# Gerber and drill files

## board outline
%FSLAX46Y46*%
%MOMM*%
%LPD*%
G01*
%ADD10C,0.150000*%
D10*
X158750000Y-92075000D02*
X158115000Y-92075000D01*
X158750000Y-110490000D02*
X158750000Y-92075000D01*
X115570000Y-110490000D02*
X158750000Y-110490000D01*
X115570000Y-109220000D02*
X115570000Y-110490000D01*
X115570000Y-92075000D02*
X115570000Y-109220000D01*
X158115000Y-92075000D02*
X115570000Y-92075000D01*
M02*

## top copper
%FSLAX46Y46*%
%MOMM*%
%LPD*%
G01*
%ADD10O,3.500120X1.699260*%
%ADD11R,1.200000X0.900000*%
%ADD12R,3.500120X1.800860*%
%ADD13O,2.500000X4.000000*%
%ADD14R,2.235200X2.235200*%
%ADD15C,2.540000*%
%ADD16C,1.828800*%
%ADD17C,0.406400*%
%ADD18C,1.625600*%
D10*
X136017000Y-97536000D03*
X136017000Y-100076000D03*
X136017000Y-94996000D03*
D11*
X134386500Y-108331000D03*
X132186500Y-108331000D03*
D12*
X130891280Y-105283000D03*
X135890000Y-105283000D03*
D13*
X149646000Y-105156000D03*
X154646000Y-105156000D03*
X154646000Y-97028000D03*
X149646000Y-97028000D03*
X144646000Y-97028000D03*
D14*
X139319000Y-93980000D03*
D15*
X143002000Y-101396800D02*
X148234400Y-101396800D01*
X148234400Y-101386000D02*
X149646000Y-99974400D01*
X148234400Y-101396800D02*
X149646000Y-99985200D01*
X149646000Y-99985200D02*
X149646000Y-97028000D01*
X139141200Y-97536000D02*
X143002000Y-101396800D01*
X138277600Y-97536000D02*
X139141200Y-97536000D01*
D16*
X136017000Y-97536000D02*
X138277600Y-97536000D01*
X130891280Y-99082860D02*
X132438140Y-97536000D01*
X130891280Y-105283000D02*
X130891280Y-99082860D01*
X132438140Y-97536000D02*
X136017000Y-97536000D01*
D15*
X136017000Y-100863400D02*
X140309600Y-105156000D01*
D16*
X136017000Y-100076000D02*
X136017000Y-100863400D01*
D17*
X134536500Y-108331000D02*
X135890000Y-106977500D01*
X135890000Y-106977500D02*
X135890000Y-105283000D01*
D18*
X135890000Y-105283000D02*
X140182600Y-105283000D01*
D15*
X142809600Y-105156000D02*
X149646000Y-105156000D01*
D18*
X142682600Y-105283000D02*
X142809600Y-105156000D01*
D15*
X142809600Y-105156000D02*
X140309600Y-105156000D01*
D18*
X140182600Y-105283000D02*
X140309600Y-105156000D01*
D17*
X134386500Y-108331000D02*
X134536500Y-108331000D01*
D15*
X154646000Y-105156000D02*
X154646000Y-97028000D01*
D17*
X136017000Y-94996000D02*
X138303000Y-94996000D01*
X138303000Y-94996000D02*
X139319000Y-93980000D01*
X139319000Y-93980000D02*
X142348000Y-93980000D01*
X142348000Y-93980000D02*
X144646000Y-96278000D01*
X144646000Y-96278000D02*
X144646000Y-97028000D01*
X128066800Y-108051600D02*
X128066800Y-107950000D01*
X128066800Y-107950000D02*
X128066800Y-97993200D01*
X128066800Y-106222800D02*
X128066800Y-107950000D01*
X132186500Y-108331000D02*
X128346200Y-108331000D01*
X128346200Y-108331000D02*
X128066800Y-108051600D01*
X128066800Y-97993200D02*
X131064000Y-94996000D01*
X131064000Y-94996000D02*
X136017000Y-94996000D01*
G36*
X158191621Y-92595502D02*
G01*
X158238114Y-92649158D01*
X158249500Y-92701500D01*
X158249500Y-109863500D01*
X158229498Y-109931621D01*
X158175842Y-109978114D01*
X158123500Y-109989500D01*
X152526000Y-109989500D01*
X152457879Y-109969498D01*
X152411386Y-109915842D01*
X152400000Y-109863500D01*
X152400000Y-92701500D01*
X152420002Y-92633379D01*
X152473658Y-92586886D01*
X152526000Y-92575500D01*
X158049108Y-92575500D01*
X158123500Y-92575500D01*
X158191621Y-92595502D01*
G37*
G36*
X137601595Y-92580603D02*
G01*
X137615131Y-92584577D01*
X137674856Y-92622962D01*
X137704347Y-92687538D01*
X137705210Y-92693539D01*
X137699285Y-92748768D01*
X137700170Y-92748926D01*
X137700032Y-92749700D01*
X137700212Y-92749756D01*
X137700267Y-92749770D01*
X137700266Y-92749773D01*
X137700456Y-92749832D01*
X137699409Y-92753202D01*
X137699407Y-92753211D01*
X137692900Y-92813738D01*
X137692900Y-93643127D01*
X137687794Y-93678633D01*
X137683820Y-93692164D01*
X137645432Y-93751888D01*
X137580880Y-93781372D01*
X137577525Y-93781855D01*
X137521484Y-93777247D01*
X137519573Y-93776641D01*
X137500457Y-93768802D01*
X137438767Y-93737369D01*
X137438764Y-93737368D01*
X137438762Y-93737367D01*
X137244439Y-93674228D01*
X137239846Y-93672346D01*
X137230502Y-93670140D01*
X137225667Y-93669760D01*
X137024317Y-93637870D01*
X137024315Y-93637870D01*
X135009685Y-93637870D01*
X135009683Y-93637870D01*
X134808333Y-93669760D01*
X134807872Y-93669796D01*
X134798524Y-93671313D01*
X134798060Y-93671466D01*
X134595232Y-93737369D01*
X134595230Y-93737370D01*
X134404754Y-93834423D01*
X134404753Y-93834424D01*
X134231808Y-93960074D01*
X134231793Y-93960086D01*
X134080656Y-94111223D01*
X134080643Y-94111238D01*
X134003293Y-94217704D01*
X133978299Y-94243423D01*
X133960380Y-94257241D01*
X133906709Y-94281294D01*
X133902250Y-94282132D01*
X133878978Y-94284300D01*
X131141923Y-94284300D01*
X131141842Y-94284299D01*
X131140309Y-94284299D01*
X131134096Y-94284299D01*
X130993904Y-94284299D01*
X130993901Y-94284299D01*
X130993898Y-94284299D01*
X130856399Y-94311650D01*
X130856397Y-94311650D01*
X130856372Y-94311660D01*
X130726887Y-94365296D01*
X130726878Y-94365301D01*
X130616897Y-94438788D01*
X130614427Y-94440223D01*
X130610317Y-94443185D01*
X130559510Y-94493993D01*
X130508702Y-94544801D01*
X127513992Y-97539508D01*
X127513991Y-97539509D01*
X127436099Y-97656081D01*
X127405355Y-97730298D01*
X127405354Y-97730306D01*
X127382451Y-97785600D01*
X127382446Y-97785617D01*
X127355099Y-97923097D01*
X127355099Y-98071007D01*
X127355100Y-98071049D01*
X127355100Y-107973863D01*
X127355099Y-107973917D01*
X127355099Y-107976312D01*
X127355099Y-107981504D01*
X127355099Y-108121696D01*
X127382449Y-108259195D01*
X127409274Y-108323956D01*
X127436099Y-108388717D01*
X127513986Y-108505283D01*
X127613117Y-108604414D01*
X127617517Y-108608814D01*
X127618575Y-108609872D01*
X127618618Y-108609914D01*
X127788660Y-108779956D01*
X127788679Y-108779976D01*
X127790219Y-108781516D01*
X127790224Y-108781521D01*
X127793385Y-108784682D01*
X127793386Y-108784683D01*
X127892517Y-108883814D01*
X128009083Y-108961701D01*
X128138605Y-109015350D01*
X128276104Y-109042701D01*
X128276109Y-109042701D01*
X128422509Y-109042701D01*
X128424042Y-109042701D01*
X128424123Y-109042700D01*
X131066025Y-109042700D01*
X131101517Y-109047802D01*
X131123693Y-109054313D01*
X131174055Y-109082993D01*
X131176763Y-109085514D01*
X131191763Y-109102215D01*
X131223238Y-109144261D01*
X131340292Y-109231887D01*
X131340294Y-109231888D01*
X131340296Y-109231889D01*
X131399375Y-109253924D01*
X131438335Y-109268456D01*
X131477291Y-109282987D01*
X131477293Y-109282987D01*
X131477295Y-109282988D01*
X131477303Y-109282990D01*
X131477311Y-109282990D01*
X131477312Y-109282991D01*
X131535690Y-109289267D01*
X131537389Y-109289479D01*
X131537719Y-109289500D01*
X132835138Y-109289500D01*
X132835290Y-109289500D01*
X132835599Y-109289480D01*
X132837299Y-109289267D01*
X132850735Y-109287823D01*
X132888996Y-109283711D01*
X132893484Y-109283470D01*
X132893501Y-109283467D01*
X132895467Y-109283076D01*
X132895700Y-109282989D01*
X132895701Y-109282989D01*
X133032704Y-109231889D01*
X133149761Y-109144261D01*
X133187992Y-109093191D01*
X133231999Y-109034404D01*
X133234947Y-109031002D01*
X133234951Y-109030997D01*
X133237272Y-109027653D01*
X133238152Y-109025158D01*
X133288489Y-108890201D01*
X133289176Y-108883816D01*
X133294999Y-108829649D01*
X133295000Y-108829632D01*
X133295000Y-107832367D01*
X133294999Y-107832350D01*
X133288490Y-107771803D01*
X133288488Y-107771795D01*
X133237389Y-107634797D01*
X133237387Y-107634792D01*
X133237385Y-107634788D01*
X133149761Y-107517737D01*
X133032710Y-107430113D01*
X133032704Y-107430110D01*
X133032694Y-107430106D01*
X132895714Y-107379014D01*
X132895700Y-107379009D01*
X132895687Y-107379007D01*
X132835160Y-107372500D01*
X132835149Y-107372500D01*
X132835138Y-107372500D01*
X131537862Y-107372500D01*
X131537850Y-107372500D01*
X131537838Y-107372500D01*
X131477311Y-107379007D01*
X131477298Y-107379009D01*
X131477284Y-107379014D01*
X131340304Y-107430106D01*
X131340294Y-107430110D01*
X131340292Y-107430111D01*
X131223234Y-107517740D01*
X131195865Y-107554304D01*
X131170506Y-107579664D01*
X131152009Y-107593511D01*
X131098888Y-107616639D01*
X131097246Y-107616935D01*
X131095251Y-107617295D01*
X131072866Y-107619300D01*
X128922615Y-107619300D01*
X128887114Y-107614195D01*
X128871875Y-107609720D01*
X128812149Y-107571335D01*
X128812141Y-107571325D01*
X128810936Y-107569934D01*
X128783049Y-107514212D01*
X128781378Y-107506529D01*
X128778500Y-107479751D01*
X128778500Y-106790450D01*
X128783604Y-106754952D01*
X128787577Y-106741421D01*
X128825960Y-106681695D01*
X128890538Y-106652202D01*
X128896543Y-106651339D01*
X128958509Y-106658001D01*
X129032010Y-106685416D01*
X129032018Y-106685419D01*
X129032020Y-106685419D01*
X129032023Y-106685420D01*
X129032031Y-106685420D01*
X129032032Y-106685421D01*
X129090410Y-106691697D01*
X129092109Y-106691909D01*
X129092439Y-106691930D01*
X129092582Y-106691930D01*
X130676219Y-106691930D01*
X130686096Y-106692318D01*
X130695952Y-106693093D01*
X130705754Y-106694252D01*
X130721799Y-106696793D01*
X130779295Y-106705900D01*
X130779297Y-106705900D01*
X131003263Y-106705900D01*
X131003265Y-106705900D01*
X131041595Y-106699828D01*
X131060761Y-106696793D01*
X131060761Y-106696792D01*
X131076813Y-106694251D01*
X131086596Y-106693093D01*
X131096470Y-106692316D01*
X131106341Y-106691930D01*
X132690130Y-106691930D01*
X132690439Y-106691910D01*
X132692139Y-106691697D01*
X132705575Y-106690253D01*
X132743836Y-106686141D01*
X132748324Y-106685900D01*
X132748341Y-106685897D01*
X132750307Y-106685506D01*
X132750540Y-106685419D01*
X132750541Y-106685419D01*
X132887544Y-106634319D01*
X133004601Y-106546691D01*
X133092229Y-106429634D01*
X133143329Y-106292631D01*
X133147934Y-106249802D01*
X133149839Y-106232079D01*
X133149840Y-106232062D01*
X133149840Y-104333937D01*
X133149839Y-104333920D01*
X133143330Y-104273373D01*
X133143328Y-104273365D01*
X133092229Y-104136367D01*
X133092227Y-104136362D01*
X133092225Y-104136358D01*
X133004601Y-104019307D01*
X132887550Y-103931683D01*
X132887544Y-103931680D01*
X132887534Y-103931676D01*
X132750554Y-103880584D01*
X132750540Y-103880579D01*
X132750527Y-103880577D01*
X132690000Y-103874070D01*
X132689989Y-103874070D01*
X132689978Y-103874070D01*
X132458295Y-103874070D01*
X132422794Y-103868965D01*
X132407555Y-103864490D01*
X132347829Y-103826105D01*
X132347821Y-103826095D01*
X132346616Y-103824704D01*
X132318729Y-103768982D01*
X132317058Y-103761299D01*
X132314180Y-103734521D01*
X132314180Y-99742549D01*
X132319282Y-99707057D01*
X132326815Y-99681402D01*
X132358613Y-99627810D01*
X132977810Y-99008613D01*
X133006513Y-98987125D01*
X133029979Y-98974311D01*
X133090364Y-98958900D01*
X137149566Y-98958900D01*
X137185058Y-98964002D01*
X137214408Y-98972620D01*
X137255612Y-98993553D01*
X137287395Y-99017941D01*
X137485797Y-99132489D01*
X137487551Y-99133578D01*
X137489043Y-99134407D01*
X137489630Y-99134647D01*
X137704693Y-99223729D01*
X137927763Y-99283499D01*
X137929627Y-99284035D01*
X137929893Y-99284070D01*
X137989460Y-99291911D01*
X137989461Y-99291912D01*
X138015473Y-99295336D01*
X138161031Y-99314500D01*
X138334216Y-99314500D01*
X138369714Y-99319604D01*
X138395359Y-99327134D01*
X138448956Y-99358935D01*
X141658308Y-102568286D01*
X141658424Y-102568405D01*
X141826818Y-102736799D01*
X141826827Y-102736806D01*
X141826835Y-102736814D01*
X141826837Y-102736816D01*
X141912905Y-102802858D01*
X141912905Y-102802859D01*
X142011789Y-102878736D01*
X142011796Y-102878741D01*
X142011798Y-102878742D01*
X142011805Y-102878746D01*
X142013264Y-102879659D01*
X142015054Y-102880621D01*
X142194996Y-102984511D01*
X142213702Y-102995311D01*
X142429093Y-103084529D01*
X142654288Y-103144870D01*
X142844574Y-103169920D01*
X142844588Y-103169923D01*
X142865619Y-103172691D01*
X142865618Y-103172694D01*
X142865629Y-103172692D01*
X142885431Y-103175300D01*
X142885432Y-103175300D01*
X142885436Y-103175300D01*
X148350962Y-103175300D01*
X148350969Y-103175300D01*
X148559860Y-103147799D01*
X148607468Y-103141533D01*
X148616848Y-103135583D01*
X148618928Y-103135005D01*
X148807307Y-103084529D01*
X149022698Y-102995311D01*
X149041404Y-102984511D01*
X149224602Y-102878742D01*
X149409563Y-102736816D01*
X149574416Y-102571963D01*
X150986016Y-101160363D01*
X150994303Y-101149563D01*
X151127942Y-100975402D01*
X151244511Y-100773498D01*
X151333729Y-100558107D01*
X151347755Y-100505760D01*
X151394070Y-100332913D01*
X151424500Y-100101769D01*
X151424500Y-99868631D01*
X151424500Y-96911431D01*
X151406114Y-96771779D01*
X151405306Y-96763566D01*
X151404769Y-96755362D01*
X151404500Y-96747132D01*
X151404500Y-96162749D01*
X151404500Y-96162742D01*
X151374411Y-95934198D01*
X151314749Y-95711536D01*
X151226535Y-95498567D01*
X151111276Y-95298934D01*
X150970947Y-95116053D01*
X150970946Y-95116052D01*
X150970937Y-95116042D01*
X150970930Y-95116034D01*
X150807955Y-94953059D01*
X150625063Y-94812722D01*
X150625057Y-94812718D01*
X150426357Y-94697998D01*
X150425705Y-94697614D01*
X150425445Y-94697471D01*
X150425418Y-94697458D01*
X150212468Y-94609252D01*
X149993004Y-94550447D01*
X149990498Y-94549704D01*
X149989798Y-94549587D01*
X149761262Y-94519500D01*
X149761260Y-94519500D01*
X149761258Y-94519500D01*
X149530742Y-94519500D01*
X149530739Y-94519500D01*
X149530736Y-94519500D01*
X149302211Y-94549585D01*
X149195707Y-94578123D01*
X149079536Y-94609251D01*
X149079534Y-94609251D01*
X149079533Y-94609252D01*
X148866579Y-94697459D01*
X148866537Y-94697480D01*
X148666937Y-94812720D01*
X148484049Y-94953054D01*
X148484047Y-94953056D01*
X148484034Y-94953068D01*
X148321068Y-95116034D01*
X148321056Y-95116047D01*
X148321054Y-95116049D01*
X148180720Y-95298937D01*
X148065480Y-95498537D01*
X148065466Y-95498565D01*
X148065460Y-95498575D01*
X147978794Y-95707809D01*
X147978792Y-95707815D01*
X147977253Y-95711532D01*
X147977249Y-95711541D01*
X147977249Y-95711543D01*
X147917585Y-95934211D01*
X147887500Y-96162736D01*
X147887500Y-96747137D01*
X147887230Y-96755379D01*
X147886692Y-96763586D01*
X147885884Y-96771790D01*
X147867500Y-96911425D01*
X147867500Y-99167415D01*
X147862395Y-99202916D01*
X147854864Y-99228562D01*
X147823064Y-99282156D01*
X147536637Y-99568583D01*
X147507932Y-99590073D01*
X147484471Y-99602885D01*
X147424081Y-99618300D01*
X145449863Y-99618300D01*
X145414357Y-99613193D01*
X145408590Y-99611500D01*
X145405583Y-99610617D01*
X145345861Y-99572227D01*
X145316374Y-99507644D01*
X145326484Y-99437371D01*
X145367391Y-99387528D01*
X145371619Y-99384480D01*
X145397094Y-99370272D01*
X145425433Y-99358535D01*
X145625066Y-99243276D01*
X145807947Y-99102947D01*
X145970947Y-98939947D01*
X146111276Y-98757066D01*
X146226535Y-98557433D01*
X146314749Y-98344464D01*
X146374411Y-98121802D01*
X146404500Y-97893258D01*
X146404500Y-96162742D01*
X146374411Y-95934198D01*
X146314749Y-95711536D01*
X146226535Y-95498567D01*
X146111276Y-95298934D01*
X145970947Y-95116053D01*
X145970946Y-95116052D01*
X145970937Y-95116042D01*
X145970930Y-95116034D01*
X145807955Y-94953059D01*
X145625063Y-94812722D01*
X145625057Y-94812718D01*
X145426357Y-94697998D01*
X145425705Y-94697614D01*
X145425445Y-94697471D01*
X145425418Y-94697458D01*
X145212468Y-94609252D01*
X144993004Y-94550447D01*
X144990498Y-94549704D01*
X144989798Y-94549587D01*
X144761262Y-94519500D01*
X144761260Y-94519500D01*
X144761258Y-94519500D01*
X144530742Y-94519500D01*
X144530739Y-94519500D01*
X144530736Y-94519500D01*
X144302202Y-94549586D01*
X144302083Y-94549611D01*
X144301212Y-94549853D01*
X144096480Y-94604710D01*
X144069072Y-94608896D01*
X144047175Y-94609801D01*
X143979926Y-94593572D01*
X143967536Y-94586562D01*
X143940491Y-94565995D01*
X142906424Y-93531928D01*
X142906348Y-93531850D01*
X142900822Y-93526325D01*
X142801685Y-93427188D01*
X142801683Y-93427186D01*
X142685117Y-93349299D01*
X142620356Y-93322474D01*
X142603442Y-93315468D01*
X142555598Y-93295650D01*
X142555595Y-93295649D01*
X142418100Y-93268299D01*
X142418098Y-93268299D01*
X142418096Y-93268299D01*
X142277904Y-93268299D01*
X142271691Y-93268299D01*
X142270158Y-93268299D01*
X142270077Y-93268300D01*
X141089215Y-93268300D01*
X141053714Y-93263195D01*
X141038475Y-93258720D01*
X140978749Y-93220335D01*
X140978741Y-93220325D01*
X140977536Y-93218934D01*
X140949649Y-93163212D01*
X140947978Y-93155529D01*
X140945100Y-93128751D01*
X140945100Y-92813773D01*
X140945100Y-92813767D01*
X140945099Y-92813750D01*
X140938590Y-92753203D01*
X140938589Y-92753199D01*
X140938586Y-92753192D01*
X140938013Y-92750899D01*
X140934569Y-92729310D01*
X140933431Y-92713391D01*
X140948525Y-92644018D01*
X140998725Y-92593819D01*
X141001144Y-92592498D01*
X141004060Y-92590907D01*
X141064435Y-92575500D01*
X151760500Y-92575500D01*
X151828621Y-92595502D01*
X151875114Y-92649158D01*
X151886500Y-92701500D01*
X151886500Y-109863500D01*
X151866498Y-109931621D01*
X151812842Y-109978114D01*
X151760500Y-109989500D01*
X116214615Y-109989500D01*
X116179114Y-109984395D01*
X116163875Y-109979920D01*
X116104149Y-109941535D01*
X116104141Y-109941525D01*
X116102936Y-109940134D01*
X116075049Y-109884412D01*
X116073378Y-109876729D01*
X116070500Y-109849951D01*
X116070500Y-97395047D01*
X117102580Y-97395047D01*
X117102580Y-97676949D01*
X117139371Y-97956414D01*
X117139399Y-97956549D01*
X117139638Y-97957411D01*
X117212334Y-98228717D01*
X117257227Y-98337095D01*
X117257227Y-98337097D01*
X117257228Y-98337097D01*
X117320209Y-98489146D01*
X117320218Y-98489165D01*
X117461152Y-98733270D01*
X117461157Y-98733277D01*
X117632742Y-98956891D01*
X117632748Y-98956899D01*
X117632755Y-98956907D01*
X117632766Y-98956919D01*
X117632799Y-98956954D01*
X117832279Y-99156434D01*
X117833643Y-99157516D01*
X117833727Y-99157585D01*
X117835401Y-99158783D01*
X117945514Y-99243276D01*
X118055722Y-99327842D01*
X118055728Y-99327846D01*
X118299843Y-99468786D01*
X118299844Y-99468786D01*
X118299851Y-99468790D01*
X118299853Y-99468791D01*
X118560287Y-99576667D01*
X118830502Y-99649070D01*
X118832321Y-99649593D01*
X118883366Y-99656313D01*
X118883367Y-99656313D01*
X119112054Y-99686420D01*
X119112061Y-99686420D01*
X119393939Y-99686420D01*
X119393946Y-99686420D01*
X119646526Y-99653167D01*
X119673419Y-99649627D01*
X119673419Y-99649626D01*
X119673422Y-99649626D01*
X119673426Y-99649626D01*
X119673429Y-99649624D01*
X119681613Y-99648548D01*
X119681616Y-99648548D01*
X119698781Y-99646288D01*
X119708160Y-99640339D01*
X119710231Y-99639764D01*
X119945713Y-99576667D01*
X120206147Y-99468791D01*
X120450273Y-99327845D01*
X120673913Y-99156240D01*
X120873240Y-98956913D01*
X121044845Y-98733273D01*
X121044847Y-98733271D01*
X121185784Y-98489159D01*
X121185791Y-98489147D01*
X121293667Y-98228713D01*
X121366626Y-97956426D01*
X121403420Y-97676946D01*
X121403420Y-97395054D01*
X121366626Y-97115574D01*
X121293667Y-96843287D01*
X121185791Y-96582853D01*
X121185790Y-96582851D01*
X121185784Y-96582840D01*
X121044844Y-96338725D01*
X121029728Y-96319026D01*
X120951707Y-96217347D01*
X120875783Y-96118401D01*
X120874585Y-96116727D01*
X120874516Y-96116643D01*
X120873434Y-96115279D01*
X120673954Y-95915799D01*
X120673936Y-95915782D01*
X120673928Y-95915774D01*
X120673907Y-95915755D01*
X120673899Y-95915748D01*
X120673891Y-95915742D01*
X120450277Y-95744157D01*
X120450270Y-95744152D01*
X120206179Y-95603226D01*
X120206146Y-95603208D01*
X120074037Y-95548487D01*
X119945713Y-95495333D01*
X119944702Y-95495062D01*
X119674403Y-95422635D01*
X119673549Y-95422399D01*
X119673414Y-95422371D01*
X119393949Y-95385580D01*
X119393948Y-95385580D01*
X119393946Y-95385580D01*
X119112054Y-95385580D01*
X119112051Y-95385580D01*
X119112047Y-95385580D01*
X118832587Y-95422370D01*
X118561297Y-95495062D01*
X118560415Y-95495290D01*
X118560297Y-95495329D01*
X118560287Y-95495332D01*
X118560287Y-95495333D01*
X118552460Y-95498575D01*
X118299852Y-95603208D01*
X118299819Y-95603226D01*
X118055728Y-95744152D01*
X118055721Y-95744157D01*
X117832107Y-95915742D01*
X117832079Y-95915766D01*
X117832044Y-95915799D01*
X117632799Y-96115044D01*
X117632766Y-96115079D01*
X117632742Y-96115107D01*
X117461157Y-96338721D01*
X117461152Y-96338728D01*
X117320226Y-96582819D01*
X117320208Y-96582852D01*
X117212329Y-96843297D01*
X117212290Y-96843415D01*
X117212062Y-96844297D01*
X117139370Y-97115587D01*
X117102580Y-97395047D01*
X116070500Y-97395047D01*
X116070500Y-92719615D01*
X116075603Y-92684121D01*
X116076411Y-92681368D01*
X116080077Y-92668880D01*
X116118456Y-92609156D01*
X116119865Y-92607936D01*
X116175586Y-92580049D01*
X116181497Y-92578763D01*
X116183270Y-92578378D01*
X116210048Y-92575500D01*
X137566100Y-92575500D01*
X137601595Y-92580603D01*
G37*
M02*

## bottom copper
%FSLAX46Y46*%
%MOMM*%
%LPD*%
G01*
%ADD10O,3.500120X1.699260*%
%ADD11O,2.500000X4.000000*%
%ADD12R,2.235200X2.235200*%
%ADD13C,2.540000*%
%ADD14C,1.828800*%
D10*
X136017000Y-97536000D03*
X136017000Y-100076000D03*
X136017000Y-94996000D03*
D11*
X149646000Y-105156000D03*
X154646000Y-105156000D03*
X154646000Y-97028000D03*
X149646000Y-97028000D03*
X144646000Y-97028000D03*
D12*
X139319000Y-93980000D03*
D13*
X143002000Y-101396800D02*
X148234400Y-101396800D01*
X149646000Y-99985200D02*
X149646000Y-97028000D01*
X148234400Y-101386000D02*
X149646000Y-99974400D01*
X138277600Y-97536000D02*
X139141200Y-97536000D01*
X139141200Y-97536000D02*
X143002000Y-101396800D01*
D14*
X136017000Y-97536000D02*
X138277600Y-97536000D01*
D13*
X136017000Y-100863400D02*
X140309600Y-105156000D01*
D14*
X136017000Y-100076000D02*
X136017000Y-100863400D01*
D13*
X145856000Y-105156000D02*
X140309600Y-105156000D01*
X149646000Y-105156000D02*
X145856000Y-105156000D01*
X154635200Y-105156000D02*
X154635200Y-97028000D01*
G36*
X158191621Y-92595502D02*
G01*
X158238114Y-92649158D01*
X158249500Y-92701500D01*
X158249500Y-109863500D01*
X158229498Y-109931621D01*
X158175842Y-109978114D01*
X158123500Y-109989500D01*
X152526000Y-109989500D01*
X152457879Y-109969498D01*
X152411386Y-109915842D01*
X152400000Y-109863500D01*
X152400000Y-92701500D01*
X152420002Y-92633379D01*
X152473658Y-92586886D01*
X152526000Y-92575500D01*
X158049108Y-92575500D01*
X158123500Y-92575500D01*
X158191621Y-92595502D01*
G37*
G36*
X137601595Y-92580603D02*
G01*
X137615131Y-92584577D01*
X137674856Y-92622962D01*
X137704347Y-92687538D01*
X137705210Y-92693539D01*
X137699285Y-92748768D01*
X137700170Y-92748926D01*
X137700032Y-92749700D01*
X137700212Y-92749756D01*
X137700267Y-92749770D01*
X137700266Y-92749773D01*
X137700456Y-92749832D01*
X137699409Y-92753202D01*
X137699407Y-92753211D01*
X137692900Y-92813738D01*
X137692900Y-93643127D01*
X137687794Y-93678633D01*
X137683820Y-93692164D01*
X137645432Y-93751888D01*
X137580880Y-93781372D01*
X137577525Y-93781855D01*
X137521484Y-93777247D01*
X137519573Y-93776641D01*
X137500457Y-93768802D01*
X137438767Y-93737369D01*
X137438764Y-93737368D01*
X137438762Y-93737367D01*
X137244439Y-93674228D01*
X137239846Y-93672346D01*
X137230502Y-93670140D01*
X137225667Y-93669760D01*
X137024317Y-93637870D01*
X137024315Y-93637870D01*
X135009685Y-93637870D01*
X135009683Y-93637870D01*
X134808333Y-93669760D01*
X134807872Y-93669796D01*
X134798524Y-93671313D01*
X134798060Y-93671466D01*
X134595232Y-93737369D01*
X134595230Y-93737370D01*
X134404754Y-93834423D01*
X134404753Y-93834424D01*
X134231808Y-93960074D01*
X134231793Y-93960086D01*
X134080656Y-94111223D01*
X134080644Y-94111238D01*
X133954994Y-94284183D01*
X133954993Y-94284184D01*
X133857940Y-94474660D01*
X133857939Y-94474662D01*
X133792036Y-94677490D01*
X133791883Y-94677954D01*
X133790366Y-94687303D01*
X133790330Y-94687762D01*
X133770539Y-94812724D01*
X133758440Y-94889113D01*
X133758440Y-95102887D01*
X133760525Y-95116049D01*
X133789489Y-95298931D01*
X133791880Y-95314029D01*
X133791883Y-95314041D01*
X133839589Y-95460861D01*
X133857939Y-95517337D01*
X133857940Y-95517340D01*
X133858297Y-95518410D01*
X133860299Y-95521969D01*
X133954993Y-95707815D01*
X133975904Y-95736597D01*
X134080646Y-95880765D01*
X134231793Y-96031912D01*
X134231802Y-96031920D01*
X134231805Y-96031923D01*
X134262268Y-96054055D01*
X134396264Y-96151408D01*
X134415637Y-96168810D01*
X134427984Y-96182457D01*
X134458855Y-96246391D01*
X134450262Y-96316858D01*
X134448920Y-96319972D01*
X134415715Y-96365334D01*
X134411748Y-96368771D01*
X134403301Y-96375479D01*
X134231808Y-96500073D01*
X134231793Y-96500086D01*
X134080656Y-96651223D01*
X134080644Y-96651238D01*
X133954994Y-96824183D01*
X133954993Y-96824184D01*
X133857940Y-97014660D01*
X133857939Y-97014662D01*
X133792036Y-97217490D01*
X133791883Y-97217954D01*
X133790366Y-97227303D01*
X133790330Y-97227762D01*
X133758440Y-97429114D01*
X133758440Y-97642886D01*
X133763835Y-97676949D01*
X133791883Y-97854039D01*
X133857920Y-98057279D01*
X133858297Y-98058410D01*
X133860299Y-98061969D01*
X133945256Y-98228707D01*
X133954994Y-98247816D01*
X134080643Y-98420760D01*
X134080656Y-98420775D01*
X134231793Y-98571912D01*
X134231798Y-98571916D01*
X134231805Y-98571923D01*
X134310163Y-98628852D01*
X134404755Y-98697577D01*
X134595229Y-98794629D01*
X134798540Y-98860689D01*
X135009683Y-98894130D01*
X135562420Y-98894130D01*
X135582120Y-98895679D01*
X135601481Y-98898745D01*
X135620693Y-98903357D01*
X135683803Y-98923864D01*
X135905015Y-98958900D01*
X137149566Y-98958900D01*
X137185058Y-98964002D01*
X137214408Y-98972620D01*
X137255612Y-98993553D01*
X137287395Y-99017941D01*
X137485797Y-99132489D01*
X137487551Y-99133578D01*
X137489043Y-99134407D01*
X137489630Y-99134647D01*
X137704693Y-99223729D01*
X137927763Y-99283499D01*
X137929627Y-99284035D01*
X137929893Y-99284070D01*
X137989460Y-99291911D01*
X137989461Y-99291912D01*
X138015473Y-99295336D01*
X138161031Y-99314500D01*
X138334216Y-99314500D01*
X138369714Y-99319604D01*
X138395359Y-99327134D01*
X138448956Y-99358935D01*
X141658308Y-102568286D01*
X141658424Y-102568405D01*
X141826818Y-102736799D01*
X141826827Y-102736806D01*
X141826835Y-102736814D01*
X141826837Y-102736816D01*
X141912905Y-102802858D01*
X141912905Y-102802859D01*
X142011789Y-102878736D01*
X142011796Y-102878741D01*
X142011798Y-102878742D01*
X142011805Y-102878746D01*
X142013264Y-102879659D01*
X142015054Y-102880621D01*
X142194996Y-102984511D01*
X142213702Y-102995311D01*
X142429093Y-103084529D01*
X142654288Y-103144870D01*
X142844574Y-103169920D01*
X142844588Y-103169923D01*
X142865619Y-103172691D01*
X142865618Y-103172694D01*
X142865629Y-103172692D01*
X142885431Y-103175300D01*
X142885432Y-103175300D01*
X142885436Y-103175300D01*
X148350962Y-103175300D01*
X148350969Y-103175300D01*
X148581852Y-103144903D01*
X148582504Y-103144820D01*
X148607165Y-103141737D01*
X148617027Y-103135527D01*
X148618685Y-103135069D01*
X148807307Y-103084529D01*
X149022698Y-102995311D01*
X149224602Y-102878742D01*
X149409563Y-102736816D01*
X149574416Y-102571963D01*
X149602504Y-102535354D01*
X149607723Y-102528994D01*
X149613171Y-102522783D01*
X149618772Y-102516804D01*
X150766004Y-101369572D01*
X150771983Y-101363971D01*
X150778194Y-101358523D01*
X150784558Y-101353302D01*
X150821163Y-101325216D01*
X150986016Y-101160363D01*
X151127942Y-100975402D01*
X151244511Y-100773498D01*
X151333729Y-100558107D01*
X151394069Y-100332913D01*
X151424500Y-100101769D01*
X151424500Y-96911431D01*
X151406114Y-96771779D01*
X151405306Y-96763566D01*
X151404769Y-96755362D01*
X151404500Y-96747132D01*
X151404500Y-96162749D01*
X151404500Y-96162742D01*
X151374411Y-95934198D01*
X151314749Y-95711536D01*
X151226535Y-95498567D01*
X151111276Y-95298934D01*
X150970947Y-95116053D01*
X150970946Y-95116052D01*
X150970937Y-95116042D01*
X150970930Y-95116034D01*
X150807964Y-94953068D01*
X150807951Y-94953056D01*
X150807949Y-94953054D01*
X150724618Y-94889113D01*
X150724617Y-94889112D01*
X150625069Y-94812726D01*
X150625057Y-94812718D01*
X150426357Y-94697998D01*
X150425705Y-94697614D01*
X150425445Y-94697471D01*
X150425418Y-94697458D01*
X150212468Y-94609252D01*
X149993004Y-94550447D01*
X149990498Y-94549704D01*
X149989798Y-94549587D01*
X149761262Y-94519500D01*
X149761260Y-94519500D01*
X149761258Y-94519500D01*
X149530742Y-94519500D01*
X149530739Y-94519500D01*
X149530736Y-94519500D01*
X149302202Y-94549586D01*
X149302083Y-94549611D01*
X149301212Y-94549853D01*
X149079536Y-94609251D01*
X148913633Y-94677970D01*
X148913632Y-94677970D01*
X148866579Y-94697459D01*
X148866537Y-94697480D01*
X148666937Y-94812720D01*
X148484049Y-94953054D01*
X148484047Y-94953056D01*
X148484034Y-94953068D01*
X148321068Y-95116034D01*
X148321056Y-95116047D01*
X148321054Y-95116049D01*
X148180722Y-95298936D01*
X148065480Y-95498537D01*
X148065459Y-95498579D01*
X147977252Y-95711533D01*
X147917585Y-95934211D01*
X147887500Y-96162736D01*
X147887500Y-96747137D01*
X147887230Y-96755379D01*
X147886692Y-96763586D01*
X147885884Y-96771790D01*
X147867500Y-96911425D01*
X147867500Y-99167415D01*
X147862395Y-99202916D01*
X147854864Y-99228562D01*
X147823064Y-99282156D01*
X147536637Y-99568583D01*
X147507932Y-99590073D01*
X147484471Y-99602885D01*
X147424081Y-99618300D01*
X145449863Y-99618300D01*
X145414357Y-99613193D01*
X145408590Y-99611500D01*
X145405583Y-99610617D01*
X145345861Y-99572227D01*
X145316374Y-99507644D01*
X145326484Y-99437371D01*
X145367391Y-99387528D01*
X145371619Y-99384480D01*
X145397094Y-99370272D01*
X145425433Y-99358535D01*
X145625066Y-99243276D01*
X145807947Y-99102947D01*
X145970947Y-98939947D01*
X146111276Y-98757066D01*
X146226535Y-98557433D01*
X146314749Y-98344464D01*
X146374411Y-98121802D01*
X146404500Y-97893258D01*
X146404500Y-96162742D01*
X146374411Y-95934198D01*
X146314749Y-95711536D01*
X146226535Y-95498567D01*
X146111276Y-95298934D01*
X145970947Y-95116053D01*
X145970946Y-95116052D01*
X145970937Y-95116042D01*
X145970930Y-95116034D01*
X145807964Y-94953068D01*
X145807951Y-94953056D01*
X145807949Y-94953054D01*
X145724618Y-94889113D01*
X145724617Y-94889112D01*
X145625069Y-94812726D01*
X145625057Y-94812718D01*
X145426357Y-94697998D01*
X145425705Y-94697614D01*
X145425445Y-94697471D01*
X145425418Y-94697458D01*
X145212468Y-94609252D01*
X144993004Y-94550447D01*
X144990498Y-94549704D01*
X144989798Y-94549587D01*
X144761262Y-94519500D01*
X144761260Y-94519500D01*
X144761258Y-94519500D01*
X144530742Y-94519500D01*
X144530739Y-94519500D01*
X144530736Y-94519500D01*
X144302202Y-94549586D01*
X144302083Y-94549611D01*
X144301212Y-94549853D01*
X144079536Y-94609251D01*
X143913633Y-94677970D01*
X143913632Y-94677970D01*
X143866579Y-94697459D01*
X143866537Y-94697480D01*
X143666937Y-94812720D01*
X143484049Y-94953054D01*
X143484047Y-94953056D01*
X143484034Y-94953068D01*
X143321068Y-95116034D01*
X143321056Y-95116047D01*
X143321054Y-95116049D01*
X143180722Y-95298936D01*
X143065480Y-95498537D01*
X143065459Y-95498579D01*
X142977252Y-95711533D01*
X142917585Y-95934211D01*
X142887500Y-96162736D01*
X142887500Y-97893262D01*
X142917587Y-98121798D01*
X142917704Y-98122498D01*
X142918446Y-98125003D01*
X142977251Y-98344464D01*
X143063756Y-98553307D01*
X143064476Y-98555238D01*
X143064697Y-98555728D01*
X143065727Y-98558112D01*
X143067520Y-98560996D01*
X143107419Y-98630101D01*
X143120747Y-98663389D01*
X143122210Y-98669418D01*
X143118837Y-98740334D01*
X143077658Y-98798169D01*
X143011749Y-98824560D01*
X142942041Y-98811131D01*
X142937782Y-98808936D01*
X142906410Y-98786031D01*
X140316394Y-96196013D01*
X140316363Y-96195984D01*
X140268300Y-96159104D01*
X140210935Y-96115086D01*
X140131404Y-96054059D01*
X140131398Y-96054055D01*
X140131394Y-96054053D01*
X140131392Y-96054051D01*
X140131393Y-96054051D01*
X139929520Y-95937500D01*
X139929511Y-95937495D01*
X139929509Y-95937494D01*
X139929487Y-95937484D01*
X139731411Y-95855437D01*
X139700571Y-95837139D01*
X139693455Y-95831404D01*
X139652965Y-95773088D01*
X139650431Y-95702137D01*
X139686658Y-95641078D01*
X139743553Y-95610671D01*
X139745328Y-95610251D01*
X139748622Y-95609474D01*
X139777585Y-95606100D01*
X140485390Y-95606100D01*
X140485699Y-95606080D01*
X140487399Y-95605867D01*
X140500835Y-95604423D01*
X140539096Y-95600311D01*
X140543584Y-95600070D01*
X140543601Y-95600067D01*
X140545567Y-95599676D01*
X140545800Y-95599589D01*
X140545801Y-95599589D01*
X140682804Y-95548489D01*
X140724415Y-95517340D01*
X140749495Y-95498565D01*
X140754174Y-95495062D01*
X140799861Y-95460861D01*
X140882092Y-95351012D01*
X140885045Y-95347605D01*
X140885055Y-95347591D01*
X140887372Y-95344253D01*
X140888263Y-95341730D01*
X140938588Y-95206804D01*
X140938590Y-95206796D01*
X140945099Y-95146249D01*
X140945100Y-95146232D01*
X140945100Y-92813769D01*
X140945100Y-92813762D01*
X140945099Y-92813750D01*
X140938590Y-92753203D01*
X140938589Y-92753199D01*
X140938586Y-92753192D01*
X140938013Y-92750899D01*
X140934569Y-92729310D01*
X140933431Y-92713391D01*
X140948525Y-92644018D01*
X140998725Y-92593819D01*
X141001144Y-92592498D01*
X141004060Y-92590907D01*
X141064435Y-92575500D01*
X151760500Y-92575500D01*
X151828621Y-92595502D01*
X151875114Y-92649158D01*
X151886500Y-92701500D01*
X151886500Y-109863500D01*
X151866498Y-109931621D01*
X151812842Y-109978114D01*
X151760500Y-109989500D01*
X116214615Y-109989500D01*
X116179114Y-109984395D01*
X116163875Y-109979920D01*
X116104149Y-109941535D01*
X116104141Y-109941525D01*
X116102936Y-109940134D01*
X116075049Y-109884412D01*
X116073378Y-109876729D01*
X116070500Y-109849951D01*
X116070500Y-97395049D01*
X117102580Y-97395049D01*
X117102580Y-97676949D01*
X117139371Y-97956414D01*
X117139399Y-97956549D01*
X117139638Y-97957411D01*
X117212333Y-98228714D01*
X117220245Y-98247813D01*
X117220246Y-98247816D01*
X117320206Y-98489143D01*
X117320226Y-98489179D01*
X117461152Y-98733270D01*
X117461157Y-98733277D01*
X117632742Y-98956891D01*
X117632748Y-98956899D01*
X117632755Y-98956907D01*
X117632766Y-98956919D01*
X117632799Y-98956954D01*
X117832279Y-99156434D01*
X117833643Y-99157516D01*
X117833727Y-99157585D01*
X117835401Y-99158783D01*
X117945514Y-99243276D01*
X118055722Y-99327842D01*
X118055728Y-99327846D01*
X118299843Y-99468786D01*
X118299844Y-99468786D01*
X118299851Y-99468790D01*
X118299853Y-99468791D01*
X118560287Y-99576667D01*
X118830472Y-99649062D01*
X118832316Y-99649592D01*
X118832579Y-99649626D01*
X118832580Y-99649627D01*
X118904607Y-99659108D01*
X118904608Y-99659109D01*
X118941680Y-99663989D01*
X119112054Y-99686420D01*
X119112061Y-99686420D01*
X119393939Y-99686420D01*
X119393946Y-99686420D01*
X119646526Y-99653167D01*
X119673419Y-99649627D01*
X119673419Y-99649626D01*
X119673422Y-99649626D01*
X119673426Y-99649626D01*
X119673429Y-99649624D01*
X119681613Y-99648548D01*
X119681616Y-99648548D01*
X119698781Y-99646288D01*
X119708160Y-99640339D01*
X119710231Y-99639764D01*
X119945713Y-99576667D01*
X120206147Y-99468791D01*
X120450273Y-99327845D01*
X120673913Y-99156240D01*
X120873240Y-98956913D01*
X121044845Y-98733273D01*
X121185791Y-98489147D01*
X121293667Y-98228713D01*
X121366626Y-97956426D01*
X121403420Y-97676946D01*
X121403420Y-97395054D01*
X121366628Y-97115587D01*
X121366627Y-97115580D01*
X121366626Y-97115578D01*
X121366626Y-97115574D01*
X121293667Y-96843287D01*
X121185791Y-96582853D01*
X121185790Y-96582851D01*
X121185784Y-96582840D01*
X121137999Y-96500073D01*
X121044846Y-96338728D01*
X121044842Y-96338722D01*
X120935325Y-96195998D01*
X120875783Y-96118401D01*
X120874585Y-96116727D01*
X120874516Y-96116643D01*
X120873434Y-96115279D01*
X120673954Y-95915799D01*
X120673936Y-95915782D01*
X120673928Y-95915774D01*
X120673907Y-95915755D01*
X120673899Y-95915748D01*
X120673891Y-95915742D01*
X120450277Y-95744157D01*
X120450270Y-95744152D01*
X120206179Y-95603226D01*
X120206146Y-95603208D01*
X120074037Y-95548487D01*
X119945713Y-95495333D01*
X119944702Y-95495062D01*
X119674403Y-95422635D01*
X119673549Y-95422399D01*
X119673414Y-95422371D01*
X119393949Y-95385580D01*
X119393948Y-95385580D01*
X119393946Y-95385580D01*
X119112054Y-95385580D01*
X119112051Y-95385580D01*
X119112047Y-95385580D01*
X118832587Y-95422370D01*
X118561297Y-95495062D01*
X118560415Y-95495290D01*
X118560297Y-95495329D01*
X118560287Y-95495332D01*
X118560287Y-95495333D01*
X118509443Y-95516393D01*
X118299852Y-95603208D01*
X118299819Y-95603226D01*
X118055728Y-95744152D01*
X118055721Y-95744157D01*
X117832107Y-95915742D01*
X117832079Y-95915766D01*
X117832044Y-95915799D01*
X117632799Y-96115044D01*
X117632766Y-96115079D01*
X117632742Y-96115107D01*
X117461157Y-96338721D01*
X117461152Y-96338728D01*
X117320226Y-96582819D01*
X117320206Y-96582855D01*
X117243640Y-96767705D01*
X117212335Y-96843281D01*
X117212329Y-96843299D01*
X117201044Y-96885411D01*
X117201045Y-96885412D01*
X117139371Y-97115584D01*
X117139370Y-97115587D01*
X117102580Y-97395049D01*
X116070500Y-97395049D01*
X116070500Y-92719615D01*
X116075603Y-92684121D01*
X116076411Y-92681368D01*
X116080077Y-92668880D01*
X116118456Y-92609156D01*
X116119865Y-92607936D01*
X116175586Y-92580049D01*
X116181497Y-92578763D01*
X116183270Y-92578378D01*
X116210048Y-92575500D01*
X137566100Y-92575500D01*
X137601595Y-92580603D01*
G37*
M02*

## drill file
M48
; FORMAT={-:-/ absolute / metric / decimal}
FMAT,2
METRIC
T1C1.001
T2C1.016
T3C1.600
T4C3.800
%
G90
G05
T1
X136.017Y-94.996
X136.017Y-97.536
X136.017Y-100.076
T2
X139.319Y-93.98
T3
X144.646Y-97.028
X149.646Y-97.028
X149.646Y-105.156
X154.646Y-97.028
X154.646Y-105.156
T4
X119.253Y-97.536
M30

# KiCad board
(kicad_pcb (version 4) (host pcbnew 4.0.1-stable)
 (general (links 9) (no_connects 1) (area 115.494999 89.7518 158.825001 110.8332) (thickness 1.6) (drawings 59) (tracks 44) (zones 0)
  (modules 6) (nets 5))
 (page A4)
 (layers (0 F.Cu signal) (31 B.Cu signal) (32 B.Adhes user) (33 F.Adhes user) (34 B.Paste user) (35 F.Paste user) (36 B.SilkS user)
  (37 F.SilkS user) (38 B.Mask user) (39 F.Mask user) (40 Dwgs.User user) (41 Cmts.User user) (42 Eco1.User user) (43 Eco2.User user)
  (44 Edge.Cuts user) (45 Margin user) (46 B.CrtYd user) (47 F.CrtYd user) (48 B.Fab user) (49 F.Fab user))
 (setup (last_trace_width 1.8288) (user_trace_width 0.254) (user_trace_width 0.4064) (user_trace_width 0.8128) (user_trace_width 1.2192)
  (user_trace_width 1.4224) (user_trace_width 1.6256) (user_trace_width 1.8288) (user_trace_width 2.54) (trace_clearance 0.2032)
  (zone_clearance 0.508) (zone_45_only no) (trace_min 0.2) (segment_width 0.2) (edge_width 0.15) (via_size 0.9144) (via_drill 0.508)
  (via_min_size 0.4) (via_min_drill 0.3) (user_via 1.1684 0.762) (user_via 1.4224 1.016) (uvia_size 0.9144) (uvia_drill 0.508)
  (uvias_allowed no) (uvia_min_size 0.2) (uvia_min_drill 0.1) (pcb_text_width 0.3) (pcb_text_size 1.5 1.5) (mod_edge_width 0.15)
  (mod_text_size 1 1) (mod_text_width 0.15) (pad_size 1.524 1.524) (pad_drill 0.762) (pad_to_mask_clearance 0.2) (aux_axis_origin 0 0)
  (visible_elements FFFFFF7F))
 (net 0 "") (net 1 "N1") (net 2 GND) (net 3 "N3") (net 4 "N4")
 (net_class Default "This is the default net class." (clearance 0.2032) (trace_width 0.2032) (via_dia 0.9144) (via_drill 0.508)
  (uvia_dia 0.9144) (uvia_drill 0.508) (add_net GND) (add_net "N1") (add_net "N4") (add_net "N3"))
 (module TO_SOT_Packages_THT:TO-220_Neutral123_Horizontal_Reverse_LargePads (layer F.Cu) (at 136.017 97.536 90)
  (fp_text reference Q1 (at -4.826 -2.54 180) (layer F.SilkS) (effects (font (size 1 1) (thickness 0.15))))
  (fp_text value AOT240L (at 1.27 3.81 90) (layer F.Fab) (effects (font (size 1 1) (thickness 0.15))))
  (pad 2 thru_hole oval (at 0 0 180) (size 3.50012 1.69926) (drill 1.00076) (layers *.Cu *.Mask F.SilkS) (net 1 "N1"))
  (pad 3 thru_hole oval (at -2.54 0 180) (size 3.50012 1.69926) (drill 1.00076) (layers *.Cu *.Mask F.SilkS) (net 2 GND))
  (pad 1 thru_hole oval (at 2.54 0 180) (size 3.50012 1.69926) (drill 1.00076) (layers *.Cu *.Mask F.SilkS) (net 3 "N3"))
  (pad "" np_thru_hole circle (at 0 -16.764 180) (size 3.79984 3.79984) (drill 3.79984) (layers *.Cu *.Mask F.SilkS)))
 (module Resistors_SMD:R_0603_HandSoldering (layer F.Cu) (at 133.2865 108.331 180)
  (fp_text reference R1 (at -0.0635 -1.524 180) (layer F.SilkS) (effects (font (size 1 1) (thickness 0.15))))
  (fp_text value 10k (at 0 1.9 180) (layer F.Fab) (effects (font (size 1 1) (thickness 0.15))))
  (pad 1 smd rect (at -1.1 0 180) (size 1.2 0.9) (layers F.Cu F.Paste F.Mask) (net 2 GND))
  (pad 2 smd rect (at 1.1 0 180) (size 1.2 0.9) (layers F.Cu F.Paste F.Mask) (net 3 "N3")))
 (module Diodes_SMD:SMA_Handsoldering (layer F.Cu) (at 133.39064 105.283)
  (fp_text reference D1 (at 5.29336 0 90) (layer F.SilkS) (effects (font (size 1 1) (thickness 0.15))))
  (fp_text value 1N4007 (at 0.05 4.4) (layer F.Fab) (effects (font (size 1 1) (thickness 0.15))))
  (pad 1 smd rect (at -2.49936 0) (size 3.50012 1.80086) (layers F.Cu F.Paste F.Mask) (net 1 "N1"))
  (pad 2 smd rect (at 2.49936 0) (size 3.50012 1.80086) (layers F.Cu F.Paste F.Mask) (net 2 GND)))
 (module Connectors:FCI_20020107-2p (layer F.Cu) (at 152.146 105.156)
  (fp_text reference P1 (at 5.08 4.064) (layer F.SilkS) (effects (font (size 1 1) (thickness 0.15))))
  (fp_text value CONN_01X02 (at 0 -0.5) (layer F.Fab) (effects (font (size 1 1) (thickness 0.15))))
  (pad 1 thru_hole oval (at -2.5 0 180) (size 2.5 4) (drill 1.6) (layers *.Cu *.Mask F.SilkS) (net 2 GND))
  (pad 2 thru_hole oval (at 2.5 0) (size 2.5 4) (drill 1.6) (layers *.Cu *.Mask F.SilkS) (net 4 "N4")))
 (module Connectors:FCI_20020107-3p (layer F.Cu) (at 149.646 97.028 180)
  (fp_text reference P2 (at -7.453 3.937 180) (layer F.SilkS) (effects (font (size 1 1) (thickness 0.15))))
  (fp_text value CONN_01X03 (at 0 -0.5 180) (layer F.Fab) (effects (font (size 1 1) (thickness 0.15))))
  (pad 1 thru_hole oval (at -5 0) (size 2.5 4) (drill 1.6) (layers *.Cu *.Mask F.SilkS) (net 4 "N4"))
  (pad 2 thru_hole oval (at 0 0) (size 2.5 4) (drill 1.6) (layers *.Cu *.Mask F.SilkS) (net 1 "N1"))
  (pad 3 thru_hole oval (at 5 0) (size 2.5 4) (drill 1.6) (layers *.Cu *.Mask F.SilkS) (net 3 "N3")))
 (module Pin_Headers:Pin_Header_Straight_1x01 (layer F.Cu) (at 139.319 93.98)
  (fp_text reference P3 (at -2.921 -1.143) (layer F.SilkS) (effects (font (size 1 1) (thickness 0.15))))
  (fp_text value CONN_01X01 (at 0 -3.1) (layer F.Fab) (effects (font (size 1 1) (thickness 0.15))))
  (pad 1 thru_hole rect (at 0 0) (size 2.2352 2.2352) (drill 1.016) (layers *.Cu *.Mask F.SilkS) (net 3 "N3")))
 (gr_line (start 158.75 92.075) (end 158.115 92.075) (layer Edge.Cuts) (width 0.15))
 (gr_line (start 158.75 110.49) (end 158.75 92.075) (layer Edge.Cuts) (width 0.15))
 (gr_line (start 115.57 110.49) (end 158.75 110.49) (layer Edge.Cuts) (width 0.15))
 (gr_line (start 115.57 109.22) (end 115.57 110.49) (layer Edge.Cuts) (width 0.15))
 (gr_line (start 115.57 92.075) (end 115.57 109.22) (layer Edge.Cuts) (width 0.15))
 (gr_line (start 158.115 92.075) (end 115.57 92.075) (layer Edge.Cuts) (width 0.15))
 (segment (start 143.002 101.3968) (end 148.2344 101.3968) (width 2.54) (layer F.Cu) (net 1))
 (segment (start 143.002 101.3968) (end 148.2344 101.3968) (width 2.54) (layer B.Cu) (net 1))
 (segment (start 148.2344 101.386) (end 149.646 99.9744) (width 2.54) (layer F.Cu) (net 1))
 (segment (start 148.2344 101.3968) (end 149.646 99.9852) (width 2.54) (layer F.Cu) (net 1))
 (segment (start 149.646 99.9852) (end 149.646 97.028) (width 2.54) (layer B.Cu) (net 1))
 (segment (start 148.2344 101.386) (end 149.646 99.9744) (width 2.54) (layer B.Cu) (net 1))
 (segment (start 149.646 99.9852) (end 149.646 97.028) (width 2.54) (layer F.Cu) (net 1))
 (segment (start 139.1412 97.536) (end 143.002 101.3968) (width 2.54) (layer F.Cu) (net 1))
 (segment (start 138.2776 97.536) (end 139.1412 97.536) (width 2.54) (layer B.Cu) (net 1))
 (segment (start 139.1412 97.536) (end 143.002 101.3968) (width 2.54) (layer B.Cu) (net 1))
 (segment (start 136.017 97.536) (end 138.2776 97.536) (width 1.8288) (layer B.Cu) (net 1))
 (segment (start 138.2776 97.536) (end 139.1412 97.536) (width 2.54) (layer F.Cu) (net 1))
 (segment (start 136.017 97.536) (end 138.2776 97.536) (width 1.8288) (layer F.Cu) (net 1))
 (segment (start 130.89128 99.08286) (end 132.43814 97.536) (width 1.8288) (layer F.Cu) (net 1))
 (segment (start 130.89128 105.283) (end 130.89128 99.08286) (width 1.8288) (layer F.Cu) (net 1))
 (segment (start 132.43814 97.536) (end 136.017 97.536) (width 1.8288) (layer F.Cu) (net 1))
 (segment (start 136.017 100.8634) (end 140.3096 105.156) (width 2.54) (layer F.Cu) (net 2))
 (segment (start 136.017 100.8634) (end 140.3096 105.156) (width 2.54) (layer B.Cu) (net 2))
 (segment (start 136.017 100.076) (end 136.017 100.8634) (width 1.8288) (layer F.Cu) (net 2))
 (segment (start 136.017 100.076) (end 136.017 100.8634) (width 1.8288) (layer B.Cu) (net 2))
 (segment (start 134.5365 108.331) (end 135.89 106.9775) (width 0.4064) (layer F.Cu) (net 2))
 (segment (start 135.89 106.9775) (end 135.89 105.283) (width 0.4064) (layer F.Cu) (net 2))
 (segment (start 135.89 105.283) (end 140.1826 105.283) (width 1.6256) (layer F.Cu) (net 2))
 (segment (start 142.8096 105.156) (end 149.646 105.156) (width 2.54) (layer F.Cu) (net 2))
 (segment (start 142.6826 105.283) (end 142.8096 105.156) (width 1.6256) (layer F.Cu) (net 2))
 (segment (start 142.8096 105.156) (end 140.3096 105.156) (width 2.54) (layer F.Cu) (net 2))
 (segment (start 140.1826 105.283) (end 140.3096 105.156) (width 1.6256) (layer F.Cu) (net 2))
 (segment (start 145.856 105.156) (end 140.3096 105.156) (width 2.54) (layer B.Cu) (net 2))
 (segment (start 149.646 105.156) (end 145.856 105.156) (width 2.54) (layer B.Cu) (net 2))
 (segment (start 134.3865 108.331) (end 134.5365 108.331) (width 0.4064) (layer F.Cu) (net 2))
 (segment (start 154.646 105.156) (end 154.646 97.028) (width 2.54) (layer F.Cu) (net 4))
 (segment (start 154.6352 105.156) (end 154.6352 97.028) (width 2.54) (layer B.Cu) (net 4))
 (segment (start 136.017 94.996) (end 138.303 94.996) (width 0.4064) (layer F.Cu) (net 3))
 (segment (start 138.303 94.996) (end 139.319 93.98) (width 0.4064) (layer F.Cu) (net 3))
 (segment (start 139.319 93.98) (end 142.348 93.98) (width 0.4064) (layer F.Cu) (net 3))
 (segment (start 142.348 93.98) (end 144.646 96.278) (width 0.4064) (layer F.Cu) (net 3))
 (segment (start 144.646 96.278) (end 144.646 97.028) (width 0.4064) (layer F.Cu) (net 3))
 (segment (start 128.0668 108.0516) (end 128.0668 107.95) (width 0.4064) (layer F.Cu) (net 3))
 (segment (start 128.0668 107.95) (end 128.0668 97.9932) (width 0.4064) (layer F.Cu) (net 3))
 (segment (start 128.0668 106.2228) (end 128.0668 107.95) (width 0.4064) (layer F.Cu) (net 3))
 (segment (start 132.1865 108.331) (end 128.3462 108.331) (width 0.4064) (layer F.Cu) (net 3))
 (segment (start 128.3462 108.331) (end 128.0668 108.0516) (width 0.4064) (layer F.Cu) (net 3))
 (segment (start 128.0668 97.9932) (end 131.064 94.996) (width 0.4064) (layer F.Cu) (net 3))
 (segment (start 131.064 94.996) (end 136.017 94.996) (width 0.4064) (layer F.Cu) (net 3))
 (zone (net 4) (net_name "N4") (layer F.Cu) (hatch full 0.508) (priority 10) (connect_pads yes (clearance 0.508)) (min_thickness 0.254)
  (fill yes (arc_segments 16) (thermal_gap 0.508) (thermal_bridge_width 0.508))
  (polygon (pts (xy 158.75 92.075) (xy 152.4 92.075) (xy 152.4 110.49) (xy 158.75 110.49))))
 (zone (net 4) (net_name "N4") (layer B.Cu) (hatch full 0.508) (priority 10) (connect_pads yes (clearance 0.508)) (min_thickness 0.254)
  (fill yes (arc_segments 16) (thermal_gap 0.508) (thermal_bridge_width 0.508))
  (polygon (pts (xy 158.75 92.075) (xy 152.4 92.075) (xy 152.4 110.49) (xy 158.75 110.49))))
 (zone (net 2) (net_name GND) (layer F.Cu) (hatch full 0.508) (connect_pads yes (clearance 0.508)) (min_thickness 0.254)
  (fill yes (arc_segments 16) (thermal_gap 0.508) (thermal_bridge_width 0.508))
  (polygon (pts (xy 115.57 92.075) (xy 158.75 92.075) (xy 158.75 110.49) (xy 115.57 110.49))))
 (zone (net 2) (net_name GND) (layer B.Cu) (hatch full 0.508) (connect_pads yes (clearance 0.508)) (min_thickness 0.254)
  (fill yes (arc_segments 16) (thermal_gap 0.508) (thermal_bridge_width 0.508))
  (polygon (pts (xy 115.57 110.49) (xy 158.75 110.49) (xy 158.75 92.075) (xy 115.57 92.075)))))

